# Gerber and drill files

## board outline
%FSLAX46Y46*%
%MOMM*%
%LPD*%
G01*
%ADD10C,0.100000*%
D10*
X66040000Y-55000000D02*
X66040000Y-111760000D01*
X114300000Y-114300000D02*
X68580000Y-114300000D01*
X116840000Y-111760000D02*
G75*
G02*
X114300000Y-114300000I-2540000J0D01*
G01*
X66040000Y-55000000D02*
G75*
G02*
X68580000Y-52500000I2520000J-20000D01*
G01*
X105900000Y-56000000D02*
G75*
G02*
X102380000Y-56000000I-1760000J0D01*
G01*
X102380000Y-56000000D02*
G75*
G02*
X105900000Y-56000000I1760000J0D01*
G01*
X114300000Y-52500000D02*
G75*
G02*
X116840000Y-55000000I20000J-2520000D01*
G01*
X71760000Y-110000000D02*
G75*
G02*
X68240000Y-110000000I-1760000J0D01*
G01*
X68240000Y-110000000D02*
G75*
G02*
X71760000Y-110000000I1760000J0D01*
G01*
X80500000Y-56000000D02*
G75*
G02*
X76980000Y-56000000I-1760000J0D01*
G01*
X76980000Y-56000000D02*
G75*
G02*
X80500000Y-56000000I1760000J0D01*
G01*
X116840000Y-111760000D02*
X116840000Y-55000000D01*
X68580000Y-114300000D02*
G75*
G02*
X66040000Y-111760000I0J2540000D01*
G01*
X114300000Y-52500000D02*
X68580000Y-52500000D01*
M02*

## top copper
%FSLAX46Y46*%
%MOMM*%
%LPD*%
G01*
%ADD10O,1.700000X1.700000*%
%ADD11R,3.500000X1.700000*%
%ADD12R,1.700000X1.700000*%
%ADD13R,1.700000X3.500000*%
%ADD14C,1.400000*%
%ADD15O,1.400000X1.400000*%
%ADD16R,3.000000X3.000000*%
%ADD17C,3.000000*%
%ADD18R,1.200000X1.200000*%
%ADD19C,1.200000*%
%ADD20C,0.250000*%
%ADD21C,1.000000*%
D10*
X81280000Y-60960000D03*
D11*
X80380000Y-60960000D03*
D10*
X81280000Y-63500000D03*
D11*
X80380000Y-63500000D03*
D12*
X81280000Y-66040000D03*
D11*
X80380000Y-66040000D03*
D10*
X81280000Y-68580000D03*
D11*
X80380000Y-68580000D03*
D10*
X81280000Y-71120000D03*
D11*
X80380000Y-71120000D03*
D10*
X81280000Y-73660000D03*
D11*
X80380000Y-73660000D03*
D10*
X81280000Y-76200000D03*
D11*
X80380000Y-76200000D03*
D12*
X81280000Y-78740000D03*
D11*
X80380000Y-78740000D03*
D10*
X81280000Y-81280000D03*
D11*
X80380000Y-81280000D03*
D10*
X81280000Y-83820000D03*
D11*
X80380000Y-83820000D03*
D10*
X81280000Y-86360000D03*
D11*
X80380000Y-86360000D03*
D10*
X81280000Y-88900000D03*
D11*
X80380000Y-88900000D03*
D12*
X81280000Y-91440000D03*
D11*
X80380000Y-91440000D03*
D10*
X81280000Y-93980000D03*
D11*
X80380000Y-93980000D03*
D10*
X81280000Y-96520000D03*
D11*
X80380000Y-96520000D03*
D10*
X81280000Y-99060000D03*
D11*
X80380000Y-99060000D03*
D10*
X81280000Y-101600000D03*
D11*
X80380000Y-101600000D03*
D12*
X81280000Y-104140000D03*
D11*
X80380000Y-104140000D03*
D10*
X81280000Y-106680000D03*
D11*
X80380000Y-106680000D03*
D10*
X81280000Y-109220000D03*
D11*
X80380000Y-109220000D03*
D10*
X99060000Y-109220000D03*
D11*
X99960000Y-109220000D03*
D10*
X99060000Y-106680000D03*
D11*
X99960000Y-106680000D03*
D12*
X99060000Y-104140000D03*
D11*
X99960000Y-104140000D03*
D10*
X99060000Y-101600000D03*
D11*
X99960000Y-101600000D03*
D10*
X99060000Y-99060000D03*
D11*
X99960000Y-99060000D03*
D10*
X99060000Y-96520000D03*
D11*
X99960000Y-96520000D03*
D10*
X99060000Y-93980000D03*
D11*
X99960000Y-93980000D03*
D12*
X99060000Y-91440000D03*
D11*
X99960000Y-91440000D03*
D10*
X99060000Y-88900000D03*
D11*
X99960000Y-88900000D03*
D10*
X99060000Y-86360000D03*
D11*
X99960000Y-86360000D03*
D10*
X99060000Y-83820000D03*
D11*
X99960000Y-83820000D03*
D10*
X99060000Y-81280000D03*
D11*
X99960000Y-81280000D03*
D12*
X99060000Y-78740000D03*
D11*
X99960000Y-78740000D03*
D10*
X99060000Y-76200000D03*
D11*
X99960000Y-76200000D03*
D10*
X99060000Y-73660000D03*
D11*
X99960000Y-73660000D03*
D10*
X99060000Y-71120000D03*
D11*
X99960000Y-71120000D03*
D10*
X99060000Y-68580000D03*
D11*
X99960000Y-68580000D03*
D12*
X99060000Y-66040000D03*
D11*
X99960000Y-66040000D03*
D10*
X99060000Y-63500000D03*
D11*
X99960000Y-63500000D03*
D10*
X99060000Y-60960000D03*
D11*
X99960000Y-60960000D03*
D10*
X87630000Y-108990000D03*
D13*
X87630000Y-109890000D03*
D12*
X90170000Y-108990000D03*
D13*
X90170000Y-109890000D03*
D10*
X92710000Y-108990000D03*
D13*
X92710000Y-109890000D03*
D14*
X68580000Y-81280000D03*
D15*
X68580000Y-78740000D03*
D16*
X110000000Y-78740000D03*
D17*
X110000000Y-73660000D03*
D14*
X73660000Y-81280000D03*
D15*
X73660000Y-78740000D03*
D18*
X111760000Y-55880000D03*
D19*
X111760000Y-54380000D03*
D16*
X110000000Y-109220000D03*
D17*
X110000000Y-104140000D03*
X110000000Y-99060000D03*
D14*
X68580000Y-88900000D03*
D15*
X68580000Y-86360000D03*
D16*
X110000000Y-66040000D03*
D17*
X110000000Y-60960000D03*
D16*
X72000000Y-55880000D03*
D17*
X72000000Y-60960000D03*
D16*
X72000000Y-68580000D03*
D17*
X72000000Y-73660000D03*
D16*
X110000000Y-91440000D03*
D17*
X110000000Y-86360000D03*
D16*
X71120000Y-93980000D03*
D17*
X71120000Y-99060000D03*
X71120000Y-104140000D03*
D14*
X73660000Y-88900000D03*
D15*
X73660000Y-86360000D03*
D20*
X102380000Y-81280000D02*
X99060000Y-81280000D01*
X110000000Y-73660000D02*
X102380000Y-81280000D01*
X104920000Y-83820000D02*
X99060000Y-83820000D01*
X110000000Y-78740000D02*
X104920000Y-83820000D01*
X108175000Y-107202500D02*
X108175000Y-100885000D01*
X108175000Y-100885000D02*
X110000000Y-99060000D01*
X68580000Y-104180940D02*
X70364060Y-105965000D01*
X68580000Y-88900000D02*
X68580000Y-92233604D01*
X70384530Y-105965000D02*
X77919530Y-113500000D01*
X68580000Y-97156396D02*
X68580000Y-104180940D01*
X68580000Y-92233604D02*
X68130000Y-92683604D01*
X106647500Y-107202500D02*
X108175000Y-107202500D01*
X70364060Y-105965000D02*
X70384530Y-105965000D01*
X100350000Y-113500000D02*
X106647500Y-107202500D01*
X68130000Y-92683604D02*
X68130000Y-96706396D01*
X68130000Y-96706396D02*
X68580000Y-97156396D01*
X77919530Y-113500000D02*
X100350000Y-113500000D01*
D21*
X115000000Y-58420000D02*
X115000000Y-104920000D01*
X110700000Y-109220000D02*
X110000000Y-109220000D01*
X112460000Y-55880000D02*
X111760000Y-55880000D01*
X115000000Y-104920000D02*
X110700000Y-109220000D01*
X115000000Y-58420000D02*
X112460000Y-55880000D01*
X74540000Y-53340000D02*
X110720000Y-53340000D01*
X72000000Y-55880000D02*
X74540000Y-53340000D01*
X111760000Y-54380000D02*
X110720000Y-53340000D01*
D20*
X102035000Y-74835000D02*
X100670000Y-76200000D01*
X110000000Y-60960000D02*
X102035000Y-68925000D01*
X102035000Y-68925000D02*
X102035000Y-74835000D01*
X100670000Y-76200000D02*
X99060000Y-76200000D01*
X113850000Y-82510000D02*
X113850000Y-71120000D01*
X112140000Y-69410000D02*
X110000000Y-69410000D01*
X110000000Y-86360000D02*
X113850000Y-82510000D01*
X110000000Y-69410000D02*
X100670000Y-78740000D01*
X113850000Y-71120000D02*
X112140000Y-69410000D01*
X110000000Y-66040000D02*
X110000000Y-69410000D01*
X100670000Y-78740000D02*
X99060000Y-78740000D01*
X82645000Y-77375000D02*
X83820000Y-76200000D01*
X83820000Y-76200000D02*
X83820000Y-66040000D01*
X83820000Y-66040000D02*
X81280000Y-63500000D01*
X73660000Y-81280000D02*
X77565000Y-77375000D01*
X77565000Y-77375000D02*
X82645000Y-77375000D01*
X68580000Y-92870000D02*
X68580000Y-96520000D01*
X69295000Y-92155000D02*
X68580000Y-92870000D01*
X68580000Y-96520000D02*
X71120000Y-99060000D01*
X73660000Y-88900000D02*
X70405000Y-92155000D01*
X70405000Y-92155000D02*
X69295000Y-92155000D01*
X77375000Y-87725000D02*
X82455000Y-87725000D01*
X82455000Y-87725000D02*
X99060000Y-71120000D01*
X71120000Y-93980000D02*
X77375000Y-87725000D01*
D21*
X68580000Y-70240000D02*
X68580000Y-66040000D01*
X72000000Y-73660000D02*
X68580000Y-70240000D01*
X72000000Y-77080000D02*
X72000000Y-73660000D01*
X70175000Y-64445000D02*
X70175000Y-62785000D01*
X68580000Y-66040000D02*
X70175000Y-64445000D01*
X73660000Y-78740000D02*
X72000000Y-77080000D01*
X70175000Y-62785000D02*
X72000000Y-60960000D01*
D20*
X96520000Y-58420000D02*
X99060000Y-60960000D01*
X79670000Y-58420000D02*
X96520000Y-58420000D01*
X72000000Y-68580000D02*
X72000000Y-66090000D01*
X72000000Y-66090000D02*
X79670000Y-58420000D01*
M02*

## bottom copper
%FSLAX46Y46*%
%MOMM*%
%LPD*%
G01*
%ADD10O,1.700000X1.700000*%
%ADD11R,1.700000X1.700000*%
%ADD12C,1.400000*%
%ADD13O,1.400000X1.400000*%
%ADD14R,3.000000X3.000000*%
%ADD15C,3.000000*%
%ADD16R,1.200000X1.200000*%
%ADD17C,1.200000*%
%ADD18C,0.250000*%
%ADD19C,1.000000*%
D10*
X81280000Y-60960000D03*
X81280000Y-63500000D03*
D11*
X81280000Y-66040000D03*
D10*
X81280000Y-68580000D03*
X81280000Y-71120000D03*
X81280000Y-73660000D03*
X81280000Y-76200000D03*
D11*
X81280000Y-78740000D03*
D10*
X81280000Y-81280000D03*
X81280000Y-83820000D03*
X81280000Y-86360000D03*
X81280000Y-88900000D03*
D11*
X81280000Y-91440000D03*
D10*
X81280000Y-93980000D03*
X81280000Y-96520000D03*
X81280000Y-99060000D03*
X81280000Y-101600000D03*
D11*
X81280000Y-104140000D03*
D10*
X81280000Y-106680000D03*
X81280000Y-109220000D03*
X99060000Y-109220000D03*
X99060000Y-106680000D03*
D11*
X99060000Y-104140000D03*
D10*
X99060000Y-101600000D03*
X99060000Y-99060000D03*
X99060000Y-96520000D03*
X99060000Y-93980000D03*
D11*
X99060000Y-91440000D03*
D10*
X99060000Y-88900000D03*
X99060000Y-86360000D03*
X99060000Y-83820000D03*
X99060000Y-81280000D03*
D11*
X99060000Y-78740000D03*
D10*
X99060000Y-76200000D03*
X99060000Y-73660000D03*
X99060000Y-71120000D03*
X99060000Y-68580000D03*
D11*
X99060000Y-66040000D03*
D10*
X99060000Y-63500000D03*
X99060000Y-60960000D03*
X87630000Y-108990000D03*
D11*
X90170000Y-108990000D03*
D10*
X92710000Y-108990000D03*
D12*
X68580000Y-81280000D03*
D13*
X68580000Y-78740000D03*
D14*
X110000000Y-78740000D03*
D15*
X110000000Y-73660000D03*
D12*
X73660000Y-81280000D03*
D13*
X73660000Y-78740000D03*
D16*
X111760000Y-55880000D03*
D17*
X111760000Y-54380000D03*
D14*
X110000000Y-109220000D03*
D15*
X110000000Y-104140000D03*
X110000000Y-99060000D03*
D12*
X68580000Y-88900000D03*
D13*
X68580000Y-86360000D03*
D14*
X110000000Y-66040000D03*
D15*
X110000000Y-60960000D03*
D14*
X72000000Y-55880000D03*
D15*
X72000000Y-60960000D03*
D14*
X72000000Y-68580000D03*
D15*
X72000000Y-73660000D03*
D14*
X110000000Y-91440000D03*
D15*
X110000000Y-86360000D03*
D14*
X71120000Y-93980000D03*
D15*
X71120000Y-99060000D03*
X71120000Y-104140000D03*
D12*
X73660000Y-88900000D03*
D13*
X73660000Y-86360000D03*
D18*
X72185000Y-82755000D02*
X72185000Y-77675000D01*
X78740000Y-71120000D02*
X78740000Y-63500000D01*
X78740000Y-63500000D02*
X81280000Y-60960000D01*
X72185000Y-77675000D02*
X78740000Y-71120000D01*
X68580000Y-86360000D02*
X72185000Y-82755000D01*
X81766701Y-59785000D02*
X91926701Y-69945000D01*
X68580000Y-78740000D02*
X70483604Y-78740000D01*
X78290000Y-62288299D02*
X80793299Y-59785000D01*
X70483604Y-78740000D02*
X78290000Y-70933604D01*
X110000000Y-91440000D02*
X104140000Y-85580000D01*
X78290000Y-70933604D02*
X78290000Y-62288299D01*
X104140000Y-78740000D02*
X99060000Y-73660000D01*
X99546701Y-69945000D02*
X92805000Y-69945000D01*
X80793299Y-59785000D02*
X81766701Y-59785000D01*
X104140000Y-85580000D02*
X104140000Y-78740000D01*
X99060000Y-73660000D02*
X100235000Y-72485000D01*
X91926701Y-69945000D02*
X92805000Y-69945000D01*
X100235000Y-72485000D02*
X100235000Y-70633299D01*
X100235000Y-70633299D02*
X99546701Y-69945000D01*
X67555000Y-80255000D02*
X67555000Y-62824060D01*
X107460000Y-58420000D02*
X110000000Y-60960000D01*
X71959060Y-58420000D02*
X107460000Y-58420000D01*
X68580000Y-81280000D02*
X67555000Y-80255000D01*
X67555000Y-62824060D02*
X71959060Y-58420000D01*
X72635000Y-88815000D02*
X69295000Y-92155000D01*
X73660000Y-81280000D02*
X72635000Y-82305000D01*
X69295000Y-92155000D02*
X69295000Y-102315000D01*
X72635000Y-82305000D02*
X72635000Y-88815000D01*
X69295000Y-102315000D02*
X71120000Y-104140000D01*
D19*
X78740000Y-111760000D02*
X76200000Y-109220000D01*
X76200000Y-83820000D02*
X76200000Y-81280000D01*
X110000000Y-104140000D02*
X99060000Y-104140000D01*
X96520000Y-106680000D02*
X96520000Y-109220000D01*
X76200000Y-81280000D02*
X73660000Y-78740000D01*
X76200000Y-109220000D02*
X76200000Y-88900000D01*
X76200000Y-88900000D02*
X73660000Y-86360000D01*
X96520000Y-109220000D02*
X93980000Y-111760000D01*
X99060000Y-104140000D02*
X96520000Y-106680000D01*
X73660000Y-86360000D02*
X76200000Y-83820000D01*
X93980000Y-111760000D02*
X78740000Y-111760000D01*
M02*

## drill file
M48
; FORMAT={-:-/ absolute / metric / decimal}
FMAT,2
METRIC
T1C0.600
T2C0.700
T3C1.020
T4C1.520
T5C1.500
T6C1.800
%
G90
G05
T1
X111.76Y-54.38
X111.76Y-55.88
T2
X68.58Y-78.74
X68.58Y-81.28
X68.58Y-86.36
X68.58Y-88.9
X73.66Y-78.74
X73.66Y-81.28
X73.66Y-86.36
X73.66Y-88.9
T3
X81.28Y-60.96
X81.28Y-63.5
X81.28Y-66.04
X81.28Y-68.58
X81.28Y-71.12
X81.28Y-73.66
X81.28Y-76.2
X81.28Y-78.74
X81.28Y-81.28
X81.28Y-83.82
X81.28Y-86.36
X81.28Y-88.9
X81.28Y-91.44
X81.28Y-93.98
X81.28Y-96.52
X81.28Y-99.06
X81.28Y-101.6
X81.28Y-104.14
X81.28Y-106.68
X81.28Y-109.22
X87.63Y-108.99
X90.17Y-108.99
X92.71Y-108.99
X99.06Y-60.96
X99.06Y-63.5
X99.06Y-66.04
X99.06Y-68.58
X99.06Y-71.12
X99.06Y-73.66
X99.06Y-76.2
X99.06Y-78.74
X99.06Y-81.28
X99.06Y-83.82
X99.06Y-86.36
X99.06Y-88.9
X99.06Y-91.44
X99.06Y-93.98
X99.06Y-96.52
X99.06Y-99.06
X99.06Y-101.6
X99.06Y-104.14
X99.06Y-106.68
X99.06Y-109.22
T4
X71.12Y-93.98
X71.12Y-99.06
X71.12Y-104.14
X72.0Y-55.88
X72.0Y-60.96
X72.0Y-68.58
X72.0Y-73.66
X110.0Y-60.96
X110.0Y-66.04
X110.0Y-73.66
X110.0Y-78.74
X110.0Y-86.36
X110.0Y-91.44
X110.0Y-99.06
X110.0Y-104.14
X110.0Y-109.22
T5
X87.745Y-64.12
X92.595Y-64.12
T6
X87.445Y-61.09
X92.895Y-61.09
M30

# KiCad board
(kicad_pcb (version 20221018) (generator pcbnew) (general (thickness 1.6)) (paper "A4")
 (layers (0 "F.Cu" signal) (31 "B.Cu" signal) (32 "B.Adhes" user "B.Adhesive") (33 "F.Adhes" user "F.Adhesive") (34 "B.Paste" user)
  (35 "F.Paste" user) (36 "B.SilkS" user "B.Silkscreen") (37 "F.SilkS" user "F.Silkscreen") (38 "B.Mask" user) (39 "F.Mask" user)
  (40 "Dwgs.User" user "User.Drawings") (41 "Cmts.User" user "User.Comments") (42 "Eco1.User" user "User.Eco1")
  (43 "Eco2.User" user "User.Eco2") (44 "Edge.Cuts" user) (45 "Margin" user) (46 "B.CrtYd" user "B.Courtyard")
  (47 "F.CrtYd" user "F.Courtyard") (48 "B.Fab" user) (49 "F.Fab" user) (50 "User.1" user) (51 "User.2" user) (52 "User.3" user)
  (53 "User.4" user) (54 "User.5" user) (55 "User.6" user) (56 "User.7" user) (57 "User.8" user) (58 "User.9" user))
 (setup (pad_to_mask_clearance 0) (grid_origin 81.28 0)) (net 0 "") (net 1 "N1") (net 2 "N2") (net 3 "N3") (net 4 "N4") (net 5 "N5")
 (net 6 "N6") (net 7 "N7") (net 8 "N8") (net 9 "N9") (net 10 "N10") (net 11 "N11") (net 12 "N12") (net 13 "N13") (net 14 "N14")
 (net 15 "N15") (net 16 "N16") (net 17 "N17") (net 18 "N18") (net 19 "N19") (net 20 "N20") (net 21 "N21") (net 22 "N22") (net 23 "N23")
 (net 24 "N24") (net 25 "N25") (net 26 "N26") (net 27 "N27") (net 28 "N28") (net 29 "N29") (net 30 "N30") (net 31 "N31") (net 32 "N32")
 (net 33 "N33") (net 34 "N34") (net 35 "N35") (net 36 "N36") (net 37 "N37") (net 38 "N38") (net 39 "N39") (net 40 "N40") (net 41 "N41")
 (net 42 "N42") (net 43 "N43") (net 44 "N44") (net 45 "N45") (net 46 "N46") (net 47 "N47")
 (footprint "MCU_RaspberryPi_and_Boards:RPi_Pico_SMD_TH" (layer "F.Cu") (at 90.17 85.09)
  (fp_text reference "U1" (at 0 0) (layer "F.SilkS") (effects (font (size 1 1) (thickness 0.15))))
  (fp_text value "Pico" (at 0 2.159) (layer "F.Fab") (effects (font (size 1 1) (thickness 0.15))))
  (pad "" np_thru_hole oval (at -2.725 -24) (size 1.8 1.8) (drill 1.8) (layers "*.Cu" "*.Mask"))
  (pad "" np_thru_hole oval (at -2.425 -20.97) (size 1.5 1.5) (drill 1.5) (layers "*.Cu" "*.Mask"))
  (pad "" np_thru_hole oval (at 2.425 -20.97) (size 1.5 1.5) (drill 1.5) (layers "*.Cu" "*.Mask"))
  (pad "" np_thru_hole oval (at 2.725 -24) (size 1.8 1.8) (drill 1.8) (layers "*.Cu" "*.Mask"))
  (pad "1" thru_hole oval (at -8.89 -24.13) (size 1.7 1.7) (drill 1.02) (layers "*.Cu" "*.Mask") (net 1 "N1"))
  (pad "1" smd rect (at -8.89 -24.13) (size 3.5 1.7) (drill (offset -0.9 0)) (layers "F.Cu" "F.Mask") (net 1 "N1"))
  (pad "2" thru_hole oval (at -8.89 -21.59) (size 1.7 1.7) (drill 1.02) (layers "*.Cu" "*.Mask") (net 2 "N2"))
  (pad "2" smd rect (at -8.89 -21.59) (size 3.5 1.7) (drill (offset -0.9 0)) (layers "F.Cu" "F.Mask") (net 2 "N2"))
  (pad "3" thru_hole rect (at -8.89 -19.05) (size 1.7 1.7) (drill 1.02) (layers "*.Cu" "*.Mask") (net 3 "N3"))
  (pad "3" smd rect (at -8.89 -19.05) (size 3.5 1.7) (drill (offset -0.9 0)) (layers "F.Cu" "F.Mask") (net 3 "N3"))
  (pad "4" thru_hole oval (at -8.89 -16.51) (size 1.7 1.7) (drill 1.02) (layers "*.Cu" "*.Mask") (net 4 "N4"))
  (pad "4" smd rect (at -8.89 -16.51) (size 3.5 1.7) (drill (offset -0.9 0)) (layers "F.Cu" "F.Mask") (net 4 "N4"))
  (pad "5" thru_hole oval (at -8.89 -13.97) (size 1.7 1.7) (drill 1.02) (layers "*.Cu" "*.Mask") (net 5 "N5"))
  (pad "5" smd rect (at -8.89 -13.97) (size 3.5 1.7) (drill (offset -0.9 0)) (layers "F.Cu" "F.Mask") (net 5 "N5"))
  (pad "6" thru_hole oval (at -8.89 -11.43) (size 1.7 1.7) (drill 1.02) (layers "*.Cu" "*.Mask") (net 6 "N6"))
  (pad "6" smd rect (at -8.89 -11.43) (size 3.5 1.7) (drill (offset -0.9 0)) (layers "F.Cu" "F.Mask") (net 6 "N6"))
  (pad "7" thru_hole oval (at -8.89 -8.89) (size 1.7 1.7) (drill 1.02) (layers "*.Cu" "*.Mask") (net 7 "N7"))
  (pad "7" smd rect (at -8.89 -8.89) (size 3.5 1.7) (drill (offset -0.9 0)) (layers "F.Cu" "F.Mask") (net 7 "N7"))
  (pad "8" thru_hole rect (at -8.89 -6.35) (size 1.7 1.7) (drill 1.02) (layers "*.Cu" "*.Mask") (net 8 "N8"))
  (pad "8" smd rect (at -8.89 -6.35) (size 3.5 1.7) (drill (offset -0.9 0)) (layers "F.Cu" "F.Mask") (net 8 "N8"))
  (pad "9" thru_hole oval (at -8.89 -3.81) (size 1.7 1.7) (drill 1.02) (layers "*.Cu" "*.Mask") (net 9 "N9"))
  (pad "9" smd rect (at -8.89 -3.81) (size 3.5 1.7) (drill (offset -0.9 0)) (layers "F.Cu" "F.Mask") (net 9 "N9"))
  (pad "10" thru_hole oval (at -8.89 -1.27) (size 1.7 1.7) (drill 1.02) (layers "*.Cu" "*.Mask") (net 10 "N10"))
  (pad "10" smd rect (at -8.89 -1.27) (size 3.5 1.7) (drill (offset -0.9 0)) (layers "F.Cu" "F.Mask") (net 10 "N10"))
  (pad "11" thru_hole oval (at -8.89 1.27) (size 1.7 1.7) (drill 1.02) (layers "*.Cu" "*.Mask") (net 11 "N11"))
  (pad "11" smd rect (at -8.89 1.27) (size 3.5 1.7) (drill (offset -0.9 0)) (layers "F.Cu" "F.Mask") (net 11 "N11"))
  (pad "12" thru_hole oval (at -8.89 3.81) (size 1.7 1.7) (drill 1.02) (layers "*.Cu" "*.Mask") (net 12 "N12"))
  (pad "12" smd rect (at -8.89 3.81) (size 3.5 1.7) (drill (offset -0.9 0)) (layers "F.Cu" "F.Mask") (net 12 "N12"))
  (pad "13" thru_hole rect (at -8.89 6.35) (size 1.7 1.7) (drill 1.02) (layers "*.Cu" "*.Mask") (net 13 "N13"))
  (pad "13" smd rect (at -8.89 6.35) (size 3.5 1.7) (drill (offset -0.9 0)) (layers "F.Cu" "F.Mask") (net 13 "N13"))
  (pad "14" thru_hole oval (at -8.89 8.89) (size 1.7 1.7) (drill 1.02) (layers "*.Cu" "*.Mask") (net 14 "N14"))
  (pad "14" smd rect (at -8.89 8.89) (size 3.5 1.7) (drill (offset -0.9 0)) (layers "F.Cu" "F.Mask") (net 14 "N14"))
  (pad "15" thru_hole oval (at -8.89 11.43) (size 1.7 1.7) (drill 1.02) (layers "*.Cu" "*.Mask") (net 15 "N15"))
  (pad "15" smd rect (at -8.89 11.43) (size 3.5 1.7) (drill (offset -0.9 0)) (layers "F.Cu" "F.Mask") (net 15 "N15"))
  (pad "16" thru_hole oval (at -8.89 13.97) (size 1.7 1.7) (drill 1.02) (layers "*.Cu" "*.Mask") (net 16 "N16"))
  (pad "16" smd rect (at -8.89 13.97) (size 3.5 1.7) (drill (offset -0.9 0)) (layers "F.Cu" "F.Mask") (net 16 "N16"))
  (pad "17" thru_hole oval (at -8.89 16.51) (size 1.7 1.7) (drill 1.02) (layers "*.Cu" "*.Mask") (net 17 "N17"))
  (pad "17" smd rect (at -8.89 16.51) (size 3.5 1.7) (drill (offset -0.9 0)) (layers "F.Cu" "F.Mask") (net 17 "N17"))
  (pad "18" thru_hole rect (at -8.89 19.05) (size 1.7 1.7) (drill 1.02) (layers "*.Cu" "*.Mask") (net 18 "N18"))
  (pad "18" smd rect (at -8.89 19.05) (size 3.5 1.7) (drill (offset -0.9 0)) (layers "F.Cu" "F.Mask") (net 18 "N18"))
  (pad "19" thru_hole oval (at -8.89 21.59) (size 1.7 1.7) (drill 1.02) (layers "*.Cu" "*.Mask") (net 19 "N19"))
  (pad "19" smd rect (at -8.89 21.59) (size 3.5 1.7) (drill (offset -0.9 0)) (layers "F.Cu" "F.Mask") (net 19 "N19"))
  (pad "20" thru_hole oval (at -8.89 24.13) (size 1.7 1.7) (drill 1.02) (layers "*.Cu" "*.Mask") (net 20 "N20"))
  (pad "20" smd rect (at -8.89 24.13) (size 3.5 1.7) (drill (offset -0.9 0)) (layers "F.Cu" "F.Mask") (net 20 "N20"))
  (pad "21" thru_hole oval (at 8.89 24.13) (size 1.7 1.7) (drill 1.02) (layers "*.Cu" "*.Mask") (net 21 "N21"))
  (pad "21" smd rect (at 8.89 24.13) (size 3.5 1.7) (drill (offset 0.9 0)) (layers "F.Cu" "F.Mask") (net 21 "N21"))
  (pad "22" thru_hole oval (at 8.89 21.59) (size 1.7 1.7) (drill 1.02) (layers "*.Cu" "*.Mask") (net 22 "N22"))
  (pad "22" smd rect (at 8.89 21.59) (size 3.5 1.7) (drill (offset 0.9 0)) (layers "F.Cu" "F.Mask") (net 22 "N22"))
  (pad "23" thru_hole rect (at 8.89 19.05) (size 1.7 1.7) (drill 1.02) (layers "*.Cu" "*.Mask") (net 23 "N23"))
  (pad "23" smd rect (at 8.89 19.05) (size 3.5 1.7) (drill (offset 0.9 0)) (layers "F.Cu" "F.Mask") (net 23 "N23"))
  (pad "24" thru_hole oval (at 8.89 16.51) (size 1.7 1.7) (drill 1.02) (layers "*.Cu" "*.Mask") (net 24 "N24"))
  (pad "24" smd rect (at 8.89 16.51) (size 3.5 1.7) (drill (offset 0.9 0)) (layers "F.Cu" "F.Mask") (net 24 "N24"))
  (pad "25" thru_hole oval (at 8.89 13.97) (size 1.7 1.7) (drill 1.02) (layers "*.Cu" "*.Mask") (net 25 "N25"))
  (pad "25" smd rect (at 8.89 13.97) (size 3.5 1.7) (drill (offset 0.9 0)) (layers "F.Cu" "F.Mask") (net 25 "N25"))
  (pad "26" thru_hole oval (at 8.89 11.43) (size 1.7 1.7) (drill 1.02) (layers "*.Cu" "*.Mask") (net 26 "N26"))
  (pad "26" smd rect (at 8.89 11.43) (size 3.5 1.7) (drill (offset 0.9 0)) (layers "F.Cu" "F.Mask") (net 26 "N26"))
  (pad "27" thru_hole oval (at 8.89 8.89) (size 1.7 1.7) (drill 1.02) (layers "*.Cu" "*.Mask") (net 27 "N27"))
  (pad "27" smd rect (at 8.89 8.89) (size 3.5 1.7) (drill (offset 0.9 0)) (layers "F.Cu" "F.Mask") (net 27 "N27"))
  (pad "28" thru_hole rect (at 8.89 6.35) (size 1.7 1.7) (drill 1.02) (layers "*.Cu" "*.Mask") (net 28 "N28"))
  (pad "28" smd rect (at 8.89 6.35) (size 3.5 1.7) (drill (offset 0.9 0)) (layers "F.Cu" "F.Mask") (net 28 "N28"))
  (pad "29" thru_hole oval (at 8.89 3.81) (size 1.7 1.7) (drill 1.02) (layers "*.Cu" "*.Mask") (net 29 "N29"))
  (pad "29" smd rect (at 8.89 3.81) (size 3.5 1.7) (drill (offset 0.9 0)) (layers "F.Cu" "F.Mask") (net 29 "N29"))
  (pad "30" thru_hole oval (at 8.89 1.27) (size 1.7 1.7) (drill 1.02) (layers "*.Cu" "*.Mask") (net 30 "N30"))
  (pad "30" smd rect (at 8.89 1.27) (size 3.5 1.7) (drill (offset 0.9 0)) (layers "F.Cu" "F.Mask") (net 30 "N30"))
  (pad "31" thru_hole oval (at 8.89 -1.27) (size 1.7 1.7) (drill 1.02) (layers "*.Cu" "*.Mask") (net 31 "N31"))
  (pad "31" smd rect (at 8.89 -1.27) (size 3.5 1.7) (drill (offset 0.9 0)) (layers "F.Cu" "F.Mask") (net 31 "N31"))
  (pad "32" thru_hole oval (at 8.89 -3.81) (size 1.7 1.7) (drill 1.02) (layers "*.Cu" "*.Mask") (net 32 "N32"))
  (pad "32" smd rect (at 8.89 -3.81) (size 3.5 1.7) (drill (offset 0.9 0)) (layers "F.Cu" "F.Mask") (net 32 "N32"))
  (pad "33" thru_hole rect (at 8.89 -6.35) (size 1.7 1.7) (drill 1.02) (layers "*.Cu" "*.Mask") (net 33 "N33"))
  (pad "33" smd rect (at 8.89 -6.35) (size 3.5 1.7) (drill (offset 0.9 0)) (layers "F.Cu" "F.Mask") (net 33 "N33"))
  (pad "34" thru_hole oval (at 8.89 -8.89) (size 1.7 1.7) (drill 1.02) (layers "*.Cu" "*.Mask") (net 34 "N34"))
  (pad "34" smd rect (at 8.89 -8.89) (size 3.5 1.7) (drill (offset 0.9 0)) (layers "F.Cu" "F.Mask") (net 34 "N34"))
  (pad "35" thru_hole oval (at 8.89 -11.43) (size 1.7 1.7) (drill 1.02) (layers "*.Cu" "*.Mask") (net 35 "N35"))
  (pad "35" smd rect (at 8.89 -11.43) (size 3.5 1.7) (drill (offset 0.9 0)) (layers "F.Cu" "F.Mask") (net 35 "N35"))
  (pad "36" thru_hole oval (at 8.89 -13.97) (size 1.7 1.7) (drill 1.02) (layers "*.Cu" "*.Mask") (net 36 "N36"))
  (pad "36" smd rect (at 8.89 -13.97) (size 3.5 1.7) (drill (offset 0.9 0)) (layers "F.Cu" "F.Mask") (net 36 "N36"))
  (pad "37" thru_hole oval (at 8.89 -16.51) (size 1.7 1.7) (drill 1.02) (layers "*.Cu" "*.Mask") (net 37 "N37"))
  (pad "37" smd rect (at 8.89 -16.51) (size 3.5 1.7) (drill (offset 0.9 0)) (layers "F.Cu" "F.Mask") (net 37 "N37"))
  (pad "38" thru_hole rect (at 8.89 -19.05) (size 1.7 1.7) (drill 1.02) (layers "*.Cu" "*.Mask") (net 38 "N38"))
  (pad "38" smd rect (at 8.89 -19.05) (size 3.5 1.7) (drill (offset 0.9 0)) (layers "F.Cu" "F.Mask") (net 38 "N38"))
  (pad "39" thru_hole oval (at 8.89 -21.59) (size 1.7 1.7) (drill 1.02) (layers "*.Cu" "*.Mask") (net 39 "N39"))
  (pad "39" smd rect (at 8.89 -21.59) (size 3.5 1.7) (drill (offset 0.9 0)) (layers "F.Cu" "F.Mask") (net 39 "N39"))
  (pad "40" thru_hole oval (at 8.89 -24.13) (size 1.7 1.7) (drill 1.02) (layers "*.Cu" "*.Mask") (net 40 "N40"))
  (pad "40" smd rect (at 8.89 -24.13) (size 3.5 1.7) (drill (offset 0.9 0)) (layers "F.Cu" "F.Mask") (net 40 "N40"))
  (pad "41" thru_hole oval (at -2.54 23.9) (size 1.7 1.7) (drill 1.02) (layers "*.Cu" "*.Mask") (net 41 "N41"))
  (pad "41" smd rect (at -2.54 23.9 90) (size 3.5 1.7) (drill (offset -0.9 0)) (layers "F.Cu" "F.Mask") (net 41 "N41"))
  (pad "42" thru_hole rect (at 0 23.9) (size 1.7 1.7) (drill 1.02) (layers "*.Cu" "*.Mask") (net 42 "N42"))
  (pad "42" smd rect (at 0 23.9 90) (size 3.5 1.7) (drill (offset -0.9 0)) (layers "F.Cu" "F.Mask") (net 42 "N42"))
  (pad "43" thru_hole oval (at 2.54 23.9) (size 1.7 1.7) (drill 1.02) (layers "*.Cu" "*.Mask") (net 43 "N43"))
  (pad "43" smd rect (at 2.54 23.9 90) (size 3.5 1.7) (drill (offset -0.9 0)) (layers "F.Cu" "F.Mask") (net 43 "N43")))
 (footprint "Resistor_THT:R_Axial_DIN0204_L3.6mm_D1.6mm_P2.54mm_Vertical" (layer "F.Cu") (at 68.58 81.28 90)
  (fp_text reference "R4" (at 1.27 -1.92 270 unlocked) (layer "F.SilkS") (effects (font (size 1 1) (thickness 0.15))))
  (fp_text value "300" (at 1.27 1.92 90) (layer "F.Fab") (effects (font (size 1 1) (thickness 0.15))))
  (pad "1" thru_hole circle (at 0 0 90) (size 1.4 1.4) (drill 0.7) (layers "*.Cu" "*.Mask") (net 34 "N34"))
  (pad "2" thru_hole oval (at 2.54 0 90) (size 1.4 1.4) (drill 0.7) (layers "*.Cu" "*.Mask") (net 35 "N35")))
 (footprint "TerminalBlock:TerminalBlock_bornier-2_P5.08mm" (layer "F.Cu") (at 110 78.74 90)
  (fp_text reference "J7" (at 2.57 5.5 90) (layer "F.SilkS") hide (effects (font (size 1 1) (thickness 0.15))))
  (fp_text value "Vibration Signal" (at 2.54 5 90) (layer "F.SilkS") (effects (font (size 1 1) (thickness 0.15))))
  (pad "1" thru_hole rect (at 0 0 90) (size 3 3) (drill 1.52) (layers "*.Cu" "*.Mask") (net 31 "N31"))
  (pad "2" thru_hole circle (at 5.08 0 90) (size 3 3) (drill 1.52) (layers "*.Cu" "*.Mask") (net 32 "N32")))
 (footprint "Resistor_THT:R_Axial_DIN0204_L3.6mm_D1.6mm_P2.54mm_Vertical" (layer "F.Cu") (at 73.66 81.28 90)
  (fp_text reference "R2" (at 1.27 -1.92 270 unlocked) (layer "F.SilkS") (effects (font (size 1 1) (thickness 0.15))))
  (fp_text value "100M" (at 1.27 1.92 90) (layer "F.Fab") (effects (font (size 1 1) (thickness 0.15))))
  (pad "1" thru_hole circle (at 0 0 90) (size 1.4 1.4) (drill 0.7) (layers "*.Cu" "*.Mask") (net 2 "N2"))
  (pad "2" thru_hole oval (at 2.54 0 90) (size 1.4 1.4) (drill 0.7) (layers "*.Cu" "*.Mask") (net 23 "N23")))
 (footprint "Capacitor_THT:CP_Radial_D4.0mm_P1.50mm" (layer "F.Cu") (at 111.76 55.88 90)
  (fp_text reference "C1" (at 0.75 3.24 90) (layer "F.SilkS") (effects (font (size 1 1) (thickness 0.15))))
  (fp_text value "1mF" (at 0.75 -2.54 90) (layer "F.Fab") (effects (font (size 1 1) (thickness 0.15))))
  (pad "1" thru_hole rect (at 0 0 90) (size 1.2 1.2) (drill 0.6) (layers "*.Cu" "*.Mask") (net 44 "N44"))
  (pad "2" thru_hole circle (at 1.5 0 90) (size 1.2 1.2) (drill 0.6) (layers "*.Cu" "*.Mask") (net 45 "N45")))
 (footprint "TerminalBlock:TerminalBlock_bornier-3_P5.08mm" (layer "F.Cu") (at 110 109.22 90)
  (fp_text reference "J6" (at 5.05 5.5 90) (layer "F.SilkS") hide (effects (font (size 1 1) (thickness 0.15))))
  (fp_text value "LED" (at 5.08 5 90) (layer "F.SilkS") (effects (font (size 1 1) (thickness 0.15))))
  (pad "1" thru_hole rect (at 0 0 90) (size 3 3) (drill 1.52) (layers "*.Cu" "*.Mask") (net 44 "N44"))
  (pad "2" thru_hole circle (at 5.08 0 90) (size 3 3) (drill 1.52) (layers "*.Cu" "*.Mask") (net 23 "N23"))
  (pad "3" thru_hole circle (at 10.16 0 90) (size 3 3) (drill 1.52) (layers "*.Cu" "*.Mask") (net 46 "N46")))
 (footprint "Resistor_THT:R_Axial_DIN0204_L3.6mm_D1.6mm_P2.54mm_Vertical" (layer "F.Cu") (at 68.58 88.9 90)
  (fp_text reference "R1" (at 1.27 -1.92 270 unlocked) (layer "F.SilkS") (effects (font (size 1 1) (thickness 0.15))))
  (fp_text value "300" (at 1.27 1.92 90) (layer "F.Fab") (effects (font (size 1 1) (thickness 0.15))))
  (pad "1" thru_hole circle (at 0 0 90) (size 1.4 1.4) (drill 0.7) (layers "*.Cu" "*.Mask") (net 46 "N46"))
  (pad "2" thru_hole oval (at 2.54 0 90) (size 1.4 1.4) (drill 0.7) (layers "*.Cu" "*.Mask") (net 1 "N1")))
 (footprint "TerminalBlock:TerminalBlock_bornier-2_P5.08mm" (layer "F.Cu") (at 110 66.04 90)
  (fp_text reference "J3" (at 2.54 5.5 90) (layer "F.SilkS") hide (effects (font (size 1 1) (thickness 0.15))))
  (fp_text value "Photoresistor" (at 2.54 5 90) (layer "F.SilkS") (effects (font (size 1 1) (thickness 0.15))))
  (pad "1" thru_hole rect (at 0 0 90) (size 3 3) (drill 1.52) (layers "*.Cu" "*.Mask") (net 33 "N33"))
  (pad "2" thru_hole circle (at 5.08 0 90) (size 3 3) (drill 1.52) (layers "*.Cu" "*.Mask") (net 34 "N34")))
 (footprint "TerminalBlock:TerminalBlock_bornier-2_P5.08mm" (layer "F.Cu") (at 72 55.88 -90)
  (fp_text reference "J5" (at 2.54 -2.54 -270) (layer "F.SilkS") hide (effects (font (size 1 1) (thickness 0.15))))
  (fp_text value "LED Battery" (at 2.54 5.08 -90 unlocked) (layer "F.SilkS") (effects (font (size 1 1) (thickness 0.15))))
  (pad "1" thru_hole rect (at 0 0 270) (size 3 3) (drill 1.52) (layers "*.Cu" "*.Mask") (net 45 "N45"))
  (pad "2" thru_hole circle (at 5.08 0 270) (size 3 3) (drill 1.52) (layers "*.Cu" "*.Mask") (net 23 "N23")))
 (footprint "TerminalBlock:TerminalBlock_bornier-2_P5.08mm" (layer "F.Cu") (at 72 68.58 -90)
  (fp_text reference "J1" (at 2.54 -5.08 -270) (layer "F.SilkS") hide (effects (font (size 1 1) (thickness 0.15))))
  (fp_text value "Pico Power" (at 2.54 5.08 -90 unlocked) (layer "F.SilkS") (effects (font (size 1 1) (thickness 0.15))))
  (pad "1" thru_hole rect (at 0 0 270) (size 3 3) (drill 1.52) (layers "*.Cu" "*.Mask") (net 40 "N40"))
  (pad "2" thru_hole circle (at 5.08 0 270) (size 3 3) (drill 1.52) (layers "*.Cu" "*.Mask") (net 23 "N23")))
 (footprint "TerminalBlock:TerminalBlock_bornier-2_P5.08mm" (layer "F.Cu") (at 110 91.44 90)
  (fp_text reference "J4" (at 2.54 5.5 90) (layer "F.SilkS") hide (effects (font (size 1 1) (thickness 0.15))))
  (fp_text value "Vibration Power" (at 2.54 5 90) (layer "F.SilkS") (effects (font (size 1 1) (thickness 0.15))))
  (pad "1" thru_hole rect (at 0 0 90) (size 3 3) (drill 1.52) (layers "*.Cu" "*.Mask") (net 35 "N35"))
  (pad "2" thru_hole circle (at 5.08 0 90) (size 3 3) (drill 1.52) (layers "*.Cu" "*.Mask") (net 33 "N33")))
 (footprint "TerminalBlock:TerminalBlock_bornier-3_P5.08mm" (layer "F.Cu") (at 71.12 93.98 -90)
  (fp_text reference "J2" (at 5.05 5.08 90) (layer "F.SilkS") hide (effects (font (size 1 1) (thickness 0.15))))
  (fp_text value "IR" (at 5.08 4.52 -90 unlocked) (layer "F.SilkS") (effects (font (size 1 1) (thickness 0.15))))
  (pad "1" thru_hole rect (at 0 0 270) (size 3 3) (drill 1.52) (layers "*.Cu" "*.Mask") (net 36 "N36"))
  (pad "2" thru_hole circle (at 5.08 0 270) (size 3 3) (drill 1.52) (layers "*.Cu" "*.Mask") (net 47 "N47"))
  (pad "3" thru_hole circle (at 10.16 0 270) (size 3 3) (drill 1.52) (layers "*.Cu" "*.Mask") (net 2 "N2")))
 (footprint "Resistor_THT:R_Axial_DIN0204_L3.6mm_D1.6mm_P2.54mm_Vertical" (layer "F.Cu") (at 73.66 88.9 90)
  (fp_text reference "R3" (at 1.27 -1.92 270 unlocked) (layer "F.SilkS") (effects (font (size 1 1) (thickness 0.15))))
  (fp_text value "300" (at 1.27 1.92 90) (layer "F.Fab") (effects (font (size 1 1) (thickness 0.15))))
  (pad "1" thru_hole circle (at 0 0 90) (size 1.4 1.4) (drill 0.7) (layers "*.Cu" "*.Mask") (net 47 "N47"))
  (pad "2" thru_hole oval (at 2.54 0 90) (size 1.4 1.4) (drill 0.7) (layers "*.Cu" "*.Mask") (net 23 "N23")))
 (gr_line (start 66.04 55) (end 66.04 111.76) (stroke (width 0.1) (type default)) (layer "Edge.Cuts"))
 (gr_line (start 114.3 114.3) (end 68.58 114.3) (stroke (width 0.1) (type default)) (layer "Edge.Cuts"))
 (gr_arc (start 116.84 111.76) (mid 116.096051 113.556051) (end 114.3 114.3) (stroke (width 0.1) (type default)) (layer "Edge.Cuts"))
 (gr_arc (start 66.04 55) (mid 66.792233 53.223949) (end 68.58 52.5) (stroke (width 0.1) (type default)) (layer "Edge.Cuts"))
 (gr_circle (center 104.14 56) (end 105.9 56) (stroke (width 0.1) (type default)) (fill none) (layer "Edge.Cuts"))
 (gr_arc (start 114.3 52.5) (mid 116.087767 53.223948) (end 116.84 55) (stroke (width 0.1) (type default)) (layer "Edge.Cuts"))
 (gr_circle (center 70 110) (end 71.76 110) (stroke (width 0.1) (type default)) (fill none) (layer "Edge.Cuts"))
 (gr_circle (center 78.74 56) (end 80.5 56) (stroke (width 0.1) (type default)) (fill none) (layer "Edge.Cuts"))
 (gr_line (start 116.84 111.76) (end 116.84 55) (stroke (width 0.1) (type default)) (layer "Edge.Cuts"))
 (gr_arc (start 68.58 114.3) (mid 66.783949 113.556051) (end 66.04 111.76) (stroke (width 0.1) (type default)) (layer "Edge.Cuts"))
 (gr_line (start 114.3 52.5) (end 68.58 52.5) (stroke (width 0.1) (type default)) (layer "Edge.Cuts"))
 (segment (start 72.185 82.755) (end 72.185 77.675) (width 0.25) (layer "B.Cu") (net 1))
 (segment (start 78.74 71.12) (end 78.74 63.5) (width 0.25) (layer "B.Cu") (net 1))
 (segment (start 78.74 63.5) (end 81.28 60.96) (width 0.25) (layer "B.Cu") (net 1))
 (segment (start 72.185 77.675) (end 78.74 71.12) (width 0.25) (layer "B.Cu") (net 1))
 (segment (start 68.58 86.36) (end 72.185 82.755) (width 0.25) (layer "B.Cu") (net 1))
 (segment (start 102.38 81.28) (end 99.06 81.28) (width 0.25) (layer "F.Cu") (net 32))
 (segment (start 110 73.66) (end 102.38 81.28) (width 0.25) (layer "F.Cu") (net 32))
 (segment (start 104.92 83.82) (end 99.06 83.82) (width 0.25) (layer "F.Cu") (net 31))
 (segment (start 110 78.74) (end 104.92 83.82) (width 0.25) (layer "F.Cu") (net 31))
 (segment (start 108.175 107.2025) (end 108.175 100.885) (width 0.25) (layer "F.Cu") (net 46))
 (segment (start 108.175 100.885) (end 110 99.06) (width 0.25) (layer "F.Cu") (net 46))
 (segment (start 68.58 104.18094) (end 70.36406 105.965) (width 0.25) (layer "F.Cu") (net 46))
 (segment (start 68.58 88.9) (end 68.58 92.233604) (width 0.25) (layer "F.Cu") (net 46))
 (segment (start 70.38453 105.965) (end 77.91953 113.5) (width 0.25) (layer "F.Cu") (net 46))
 (segment (start 68.58 97.156396) (end 68.58 104.18094) (width 0.25) (layer "F.Cu") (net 46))
 (segment (start 68.58 92.233604) (end 68.13 92.683604) (width 0.25) (layer "F.Cu") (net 46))
 (segment (start 106.6475 107.2025) (end 108.175 107.2025) (width 0.25) (layer "F.Cu") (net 46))
 (segment (start 70.36406 105.965) (end 70.38453 105.965) (width 0.25) (layer "F.Cu") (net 46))
 (segment (start 100.35 113.5) (end 106.6475 107.2025) (width 0.25) (layer "F.Cu") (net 46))
 (segment (start 68.13 92.683604) (end 68.13 96.706396) (width 0.25) (layer "F.Cu") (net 46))
 (segment (start 68.13 96.706396) (end 68.58 97.156396) (width 0.25) (layer "F.Cu") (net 46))
 (segment (start 77.91953 113.5) (end 100.35 113.5) (width 0.25) (layer "F.Cu") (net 46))
 (segment (start 115 58.42) (end 115 104.92) (width 1) (layer "F.Cu") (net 44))
 (segment (start 110.7 109.22) (end 110 109.22) (width 1) (layer "F.Cu") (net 44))
 (segment (start 112.46 55.88) (end 111.76 55.88) (width 1) (layer "F.Cu") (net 44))
 (segment (start 115 104.92) (end 110.7 109.22) (width 1) (layer "F.Cu") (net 44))
 (segment (start 115 58.42) (end 112.46 55.88) (width 1) (layer "F.Cu") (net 44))
 (segment (start 74.54 53.34) (end 110.72 53.34) (width 1) (layer "F.Cu") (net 45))
 (segment (start 72 55.88) (end 74.54 53.34) (width 1) (layer "F.Cu") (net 45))
 (segment (start 111.76 54.38) (end 110.72 53.34) (width 1) (layer "F.Cu") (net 45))
 (segment (start 81.766701 59.785) (end 91.926701 69.945) (width 0.25) (layer "B.Cu") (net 35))
 (segment (start 68.58 78.74) (end 70.483604 78.74) (width 0.25) (layer "B.Cu") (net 35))
 (segment (start 78.29 62.288299) (end 80.793299 59.785) (width 0.25) (layer "B.Cu") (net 35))
 (segment (start 70.483604 78.74) (end 78.29 70.933604) (width 0.25) (layer "B.Cu") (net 35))
 (segment (start 110 91.44) (end 104.14 85.58) (width 0.25) (layer "B.Cu") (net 35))
 (segment (start 78.29 70.933604) (end 78.29 62.288299) (width 0.25) (layer "B.Cu") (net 35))
 (segment (start 104.14 78.74) (end 99.06 73.66) (width 0.25) (layer "B.Cu") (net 35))
 (segment (start 99.546701 69.945) (end 92.805 69.945) (width 0.25) (layer "B.Cu") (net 35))
 (segment (start 80.793299 59.785) (end 81.766701 59.785) (width 0.25) (layer "B.Cu") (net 35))
 (segment (start 104.14 85.58) (end 104.14 78.74) (width 0.25) (layer "B.Cu") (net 35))
 (segment (start 99.06 73.66) (end 100.235 72.485) (width 0.25) (layer "B.Cu") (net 35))
 (segment (start 91.926701 69.945) (end 92.805 69.945) (width 0.25) (layer "B.Cu") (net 35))
 (segment (start 100.235 72.485) (end 100.235 70.633299) (width 0.25) (layer "B.Cu") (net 35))
 (segment (start 100.235 70.633299) (end 99.546701 69.945) (width 0.25) (layer "B.Cu") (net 35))
 (segment (start 102.035 74.835) (end 100.67 76.2) (width 0.25) (layer "F.Cu") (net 34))
 (segment (start 110 60.96) (end 102.035 68.925) (width 0.25) (layer "F.Cu") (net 34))
 (segment (start 102.035 68.925) (end 102.035 74.835) (width 0.25) (layer "F.Cu") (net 34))
 (segment (start 100.67 76.2) (end 99.06 76.2) (width 0.25) (layer "F.Cu") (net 34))
 (segment (start 67.555 80.255) (end 67.555 62.82406) (width 0.25) (layer "B.Cu") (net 34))
 (segment (start 107.46 58.42) (end 110 60.96) (width 0.25) (layer "B.Cu") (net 34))
 (segment (start 71.95906 58.42) (end 107.46 58.42) (width 0.25) (layer "B.Cu") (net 34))
 (segment (start 68.58 81.28) (end 67.555 80.255) (width 0.25) (layer "B.Cu") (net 34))
 (segment (start 67.555 62.82406) (end 71.95906 58.42) (width 0.25) (layer "B.Cu") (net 34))
 (segment (start 113.85 82.51) (end 113.85 71.12) (width 0.25) (layer "F.Cu") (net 33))
 (segment (start 112.14 69.41) (end 110 69.41) (width 0.25) (layer "F.Cu") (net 33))
 (segment (start 110 86.36) (end 113.85 82.51) (width 0.25) (layer "F.Cu") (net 33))
 (segment (start 110 69.41) (end 100.67 78.74) (width 0.25) (layer "F.Cu") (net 33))
 (segment (start 113.85 71.12) (end 112.14 69.41) (width 0.25) (layer "F.Cu") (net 33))
 (segment (start 110 66.04) (end 110 69.41) (width 0.25) (layer "F.Cu") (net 33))
 (segment (start 100.67 78.74) (end 99.06 78.74) (width 0.25) (layer "F.Cu") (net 33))
 (segment (start 82.645 77.375) (end 83.82 76.2) (width 0.25) (layer "F.Cu") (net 2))
 (segment (start 83.82 76.2) (end 83.82 66.04) (width 0.25) (layer "F.Cu") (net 2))
 (segment (start 83.82 66.04) (end 81.28 63.5) (width 0.25) (layer "F.Cu") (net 2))
 (segment (start 73.66 81.28) (end 77.565 77.375) (width 0.25) (layer "F.Cu") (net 2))
 (segment (start 77.565 77.375) (end 82.645 77.375) (width 0.25) (layer "F.Cu") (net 2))
 (segment (start 72.635 88.815) (end 69.295 92.155) (width 0.25) (layer "B.Cu") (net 2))
 (segment (start 73.66 81.28) (end 72.635 82.305) (width 0.25) (layer "B.Cu") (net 2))
 (segment (start 69.295 92.155) (end 69.295 102.315) (width 0.25) (layer "B.Cu") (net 2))
 (segment (start 72.635 82.305) (end 72.635 88.815) (width 0.25) (layer "B.Cu") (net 2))
 (segment (start 69.295 102.315) (end 71.12 104.14) (width 0.25) (layer "B.Cu") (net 2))
 (segment (start 68.58 92.87) (end 68.58 96.52) (width 0.25) (layer "F.Cu") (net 47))
 (segment (start 69.295 92.155) (end 68.58 92.87) (width 0.25) (layer "F.Cu") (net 47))
 (segment (start 68.58 96.52) (end 71.12 99.06) (width 0.25) (layer "F.Cu") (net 47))
 (segment (start 73.66 88.9) (end 70.405 92.155) (width 0.25) (layer "F.Cu") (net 47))
 (segment (start 70.405 92.155) (end 69.295 92.155) (width 0.25) (layer "F.Cu") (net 47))
 (segment (start 77.375 87.725) (end 82.455 87.725) (width 0.25) (layer "F.Cu") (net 36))
 (segment (start 82.455 87.725) (end 99.06 71.12) (width 0.25) (layer "F.Cu") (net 36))
 (segment (start 71.12 93.98) (end 77.375 87.725) (width 0.25) (layer "F.Cu") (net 36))
 (segment (start 68.58 70.24) (end 68.58 66.04) (width 1) (layer "F.Cu") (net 23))
 (segment (start 72 73.66) (end 68.58 70.24) (width 1) (layer "F.Cu") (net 23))
 (segment (start 72 77.08) (end 72 73.66) (width 1) (layer "F.Cu") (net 23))
 (segment (start 70.175 64.445) (end 70.175 62.785) (width 1) (layer "F.Cu") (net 23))
 (segment (start 68.58 66.04) (end 70.175 64.445) (width 1) (layer "F.Cu") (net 23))
 (segment (start 73.66 78.74) (end 72 77.08) (width 1) (layer "F.Cu") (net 23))
 (segment (start 70.175 62.785) (end 72 60.96) (width 1) (layer "F.Cu") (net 23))
 (segment (start 78.74 111.76) (end 76.2 109.22) (width 1) (layer "B.Cu") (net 23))
 (segment (start 76.2 83.82) (end 76.2 81.28) (width 1) (layer "B.Cu") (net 23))
 (segment (start 110 104.14) (end 99.06 104.14) (width 1) (layer "B.Cu") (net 23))
 (segment (start 96.52 106.68) (end 96.52 109.22) (width 1) (layer "B.Cu") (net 23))
 (segment (start 76.2 81.28) (end 73.66 78.74) (width 1) (layer "B.Cu") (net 23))
 (segment (start 76.2 109.22) (end 76.2 88.9) (width 1) (layer "B.Cu") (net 23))
 (segment (start 76.2 88.9) (end 73.66 86.36) (width 1) (layer "B.Cu") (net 23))
 (segment (start 96.52 109.22) (end 93.98 111.76) (width 1) (layer "B.Cu") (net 23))
 (segment (start 99.06 104.14) (end 96.52 106.68) (width 1) (layer "B.Cu") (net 23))
 (segment (start 73.66 86.36) (end 76.2 83.82) (width 1) (layer "B.Cu") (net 23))
 (segment (start 93.98 111.76) (end 78.74 111.76) (width 1) (layer "B.Cu") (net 23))
 (segment (start 96.52 58.42) (end 99.06 60.96) (width 0.25) (layer "F.Cu") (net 40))
 (segment (start 79.67 58.42) (end 96.52 58.42) (width 0.25) (layer "F.Cu") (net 40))
 (segment (start 72 68.58) (end 72 66.09) (width 0.25) (layer "F.Cu") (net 40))
 (segment (start 72 66.09) (end 79.67 58.42) (width 0.25) (layer "F.Cu") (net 40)))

